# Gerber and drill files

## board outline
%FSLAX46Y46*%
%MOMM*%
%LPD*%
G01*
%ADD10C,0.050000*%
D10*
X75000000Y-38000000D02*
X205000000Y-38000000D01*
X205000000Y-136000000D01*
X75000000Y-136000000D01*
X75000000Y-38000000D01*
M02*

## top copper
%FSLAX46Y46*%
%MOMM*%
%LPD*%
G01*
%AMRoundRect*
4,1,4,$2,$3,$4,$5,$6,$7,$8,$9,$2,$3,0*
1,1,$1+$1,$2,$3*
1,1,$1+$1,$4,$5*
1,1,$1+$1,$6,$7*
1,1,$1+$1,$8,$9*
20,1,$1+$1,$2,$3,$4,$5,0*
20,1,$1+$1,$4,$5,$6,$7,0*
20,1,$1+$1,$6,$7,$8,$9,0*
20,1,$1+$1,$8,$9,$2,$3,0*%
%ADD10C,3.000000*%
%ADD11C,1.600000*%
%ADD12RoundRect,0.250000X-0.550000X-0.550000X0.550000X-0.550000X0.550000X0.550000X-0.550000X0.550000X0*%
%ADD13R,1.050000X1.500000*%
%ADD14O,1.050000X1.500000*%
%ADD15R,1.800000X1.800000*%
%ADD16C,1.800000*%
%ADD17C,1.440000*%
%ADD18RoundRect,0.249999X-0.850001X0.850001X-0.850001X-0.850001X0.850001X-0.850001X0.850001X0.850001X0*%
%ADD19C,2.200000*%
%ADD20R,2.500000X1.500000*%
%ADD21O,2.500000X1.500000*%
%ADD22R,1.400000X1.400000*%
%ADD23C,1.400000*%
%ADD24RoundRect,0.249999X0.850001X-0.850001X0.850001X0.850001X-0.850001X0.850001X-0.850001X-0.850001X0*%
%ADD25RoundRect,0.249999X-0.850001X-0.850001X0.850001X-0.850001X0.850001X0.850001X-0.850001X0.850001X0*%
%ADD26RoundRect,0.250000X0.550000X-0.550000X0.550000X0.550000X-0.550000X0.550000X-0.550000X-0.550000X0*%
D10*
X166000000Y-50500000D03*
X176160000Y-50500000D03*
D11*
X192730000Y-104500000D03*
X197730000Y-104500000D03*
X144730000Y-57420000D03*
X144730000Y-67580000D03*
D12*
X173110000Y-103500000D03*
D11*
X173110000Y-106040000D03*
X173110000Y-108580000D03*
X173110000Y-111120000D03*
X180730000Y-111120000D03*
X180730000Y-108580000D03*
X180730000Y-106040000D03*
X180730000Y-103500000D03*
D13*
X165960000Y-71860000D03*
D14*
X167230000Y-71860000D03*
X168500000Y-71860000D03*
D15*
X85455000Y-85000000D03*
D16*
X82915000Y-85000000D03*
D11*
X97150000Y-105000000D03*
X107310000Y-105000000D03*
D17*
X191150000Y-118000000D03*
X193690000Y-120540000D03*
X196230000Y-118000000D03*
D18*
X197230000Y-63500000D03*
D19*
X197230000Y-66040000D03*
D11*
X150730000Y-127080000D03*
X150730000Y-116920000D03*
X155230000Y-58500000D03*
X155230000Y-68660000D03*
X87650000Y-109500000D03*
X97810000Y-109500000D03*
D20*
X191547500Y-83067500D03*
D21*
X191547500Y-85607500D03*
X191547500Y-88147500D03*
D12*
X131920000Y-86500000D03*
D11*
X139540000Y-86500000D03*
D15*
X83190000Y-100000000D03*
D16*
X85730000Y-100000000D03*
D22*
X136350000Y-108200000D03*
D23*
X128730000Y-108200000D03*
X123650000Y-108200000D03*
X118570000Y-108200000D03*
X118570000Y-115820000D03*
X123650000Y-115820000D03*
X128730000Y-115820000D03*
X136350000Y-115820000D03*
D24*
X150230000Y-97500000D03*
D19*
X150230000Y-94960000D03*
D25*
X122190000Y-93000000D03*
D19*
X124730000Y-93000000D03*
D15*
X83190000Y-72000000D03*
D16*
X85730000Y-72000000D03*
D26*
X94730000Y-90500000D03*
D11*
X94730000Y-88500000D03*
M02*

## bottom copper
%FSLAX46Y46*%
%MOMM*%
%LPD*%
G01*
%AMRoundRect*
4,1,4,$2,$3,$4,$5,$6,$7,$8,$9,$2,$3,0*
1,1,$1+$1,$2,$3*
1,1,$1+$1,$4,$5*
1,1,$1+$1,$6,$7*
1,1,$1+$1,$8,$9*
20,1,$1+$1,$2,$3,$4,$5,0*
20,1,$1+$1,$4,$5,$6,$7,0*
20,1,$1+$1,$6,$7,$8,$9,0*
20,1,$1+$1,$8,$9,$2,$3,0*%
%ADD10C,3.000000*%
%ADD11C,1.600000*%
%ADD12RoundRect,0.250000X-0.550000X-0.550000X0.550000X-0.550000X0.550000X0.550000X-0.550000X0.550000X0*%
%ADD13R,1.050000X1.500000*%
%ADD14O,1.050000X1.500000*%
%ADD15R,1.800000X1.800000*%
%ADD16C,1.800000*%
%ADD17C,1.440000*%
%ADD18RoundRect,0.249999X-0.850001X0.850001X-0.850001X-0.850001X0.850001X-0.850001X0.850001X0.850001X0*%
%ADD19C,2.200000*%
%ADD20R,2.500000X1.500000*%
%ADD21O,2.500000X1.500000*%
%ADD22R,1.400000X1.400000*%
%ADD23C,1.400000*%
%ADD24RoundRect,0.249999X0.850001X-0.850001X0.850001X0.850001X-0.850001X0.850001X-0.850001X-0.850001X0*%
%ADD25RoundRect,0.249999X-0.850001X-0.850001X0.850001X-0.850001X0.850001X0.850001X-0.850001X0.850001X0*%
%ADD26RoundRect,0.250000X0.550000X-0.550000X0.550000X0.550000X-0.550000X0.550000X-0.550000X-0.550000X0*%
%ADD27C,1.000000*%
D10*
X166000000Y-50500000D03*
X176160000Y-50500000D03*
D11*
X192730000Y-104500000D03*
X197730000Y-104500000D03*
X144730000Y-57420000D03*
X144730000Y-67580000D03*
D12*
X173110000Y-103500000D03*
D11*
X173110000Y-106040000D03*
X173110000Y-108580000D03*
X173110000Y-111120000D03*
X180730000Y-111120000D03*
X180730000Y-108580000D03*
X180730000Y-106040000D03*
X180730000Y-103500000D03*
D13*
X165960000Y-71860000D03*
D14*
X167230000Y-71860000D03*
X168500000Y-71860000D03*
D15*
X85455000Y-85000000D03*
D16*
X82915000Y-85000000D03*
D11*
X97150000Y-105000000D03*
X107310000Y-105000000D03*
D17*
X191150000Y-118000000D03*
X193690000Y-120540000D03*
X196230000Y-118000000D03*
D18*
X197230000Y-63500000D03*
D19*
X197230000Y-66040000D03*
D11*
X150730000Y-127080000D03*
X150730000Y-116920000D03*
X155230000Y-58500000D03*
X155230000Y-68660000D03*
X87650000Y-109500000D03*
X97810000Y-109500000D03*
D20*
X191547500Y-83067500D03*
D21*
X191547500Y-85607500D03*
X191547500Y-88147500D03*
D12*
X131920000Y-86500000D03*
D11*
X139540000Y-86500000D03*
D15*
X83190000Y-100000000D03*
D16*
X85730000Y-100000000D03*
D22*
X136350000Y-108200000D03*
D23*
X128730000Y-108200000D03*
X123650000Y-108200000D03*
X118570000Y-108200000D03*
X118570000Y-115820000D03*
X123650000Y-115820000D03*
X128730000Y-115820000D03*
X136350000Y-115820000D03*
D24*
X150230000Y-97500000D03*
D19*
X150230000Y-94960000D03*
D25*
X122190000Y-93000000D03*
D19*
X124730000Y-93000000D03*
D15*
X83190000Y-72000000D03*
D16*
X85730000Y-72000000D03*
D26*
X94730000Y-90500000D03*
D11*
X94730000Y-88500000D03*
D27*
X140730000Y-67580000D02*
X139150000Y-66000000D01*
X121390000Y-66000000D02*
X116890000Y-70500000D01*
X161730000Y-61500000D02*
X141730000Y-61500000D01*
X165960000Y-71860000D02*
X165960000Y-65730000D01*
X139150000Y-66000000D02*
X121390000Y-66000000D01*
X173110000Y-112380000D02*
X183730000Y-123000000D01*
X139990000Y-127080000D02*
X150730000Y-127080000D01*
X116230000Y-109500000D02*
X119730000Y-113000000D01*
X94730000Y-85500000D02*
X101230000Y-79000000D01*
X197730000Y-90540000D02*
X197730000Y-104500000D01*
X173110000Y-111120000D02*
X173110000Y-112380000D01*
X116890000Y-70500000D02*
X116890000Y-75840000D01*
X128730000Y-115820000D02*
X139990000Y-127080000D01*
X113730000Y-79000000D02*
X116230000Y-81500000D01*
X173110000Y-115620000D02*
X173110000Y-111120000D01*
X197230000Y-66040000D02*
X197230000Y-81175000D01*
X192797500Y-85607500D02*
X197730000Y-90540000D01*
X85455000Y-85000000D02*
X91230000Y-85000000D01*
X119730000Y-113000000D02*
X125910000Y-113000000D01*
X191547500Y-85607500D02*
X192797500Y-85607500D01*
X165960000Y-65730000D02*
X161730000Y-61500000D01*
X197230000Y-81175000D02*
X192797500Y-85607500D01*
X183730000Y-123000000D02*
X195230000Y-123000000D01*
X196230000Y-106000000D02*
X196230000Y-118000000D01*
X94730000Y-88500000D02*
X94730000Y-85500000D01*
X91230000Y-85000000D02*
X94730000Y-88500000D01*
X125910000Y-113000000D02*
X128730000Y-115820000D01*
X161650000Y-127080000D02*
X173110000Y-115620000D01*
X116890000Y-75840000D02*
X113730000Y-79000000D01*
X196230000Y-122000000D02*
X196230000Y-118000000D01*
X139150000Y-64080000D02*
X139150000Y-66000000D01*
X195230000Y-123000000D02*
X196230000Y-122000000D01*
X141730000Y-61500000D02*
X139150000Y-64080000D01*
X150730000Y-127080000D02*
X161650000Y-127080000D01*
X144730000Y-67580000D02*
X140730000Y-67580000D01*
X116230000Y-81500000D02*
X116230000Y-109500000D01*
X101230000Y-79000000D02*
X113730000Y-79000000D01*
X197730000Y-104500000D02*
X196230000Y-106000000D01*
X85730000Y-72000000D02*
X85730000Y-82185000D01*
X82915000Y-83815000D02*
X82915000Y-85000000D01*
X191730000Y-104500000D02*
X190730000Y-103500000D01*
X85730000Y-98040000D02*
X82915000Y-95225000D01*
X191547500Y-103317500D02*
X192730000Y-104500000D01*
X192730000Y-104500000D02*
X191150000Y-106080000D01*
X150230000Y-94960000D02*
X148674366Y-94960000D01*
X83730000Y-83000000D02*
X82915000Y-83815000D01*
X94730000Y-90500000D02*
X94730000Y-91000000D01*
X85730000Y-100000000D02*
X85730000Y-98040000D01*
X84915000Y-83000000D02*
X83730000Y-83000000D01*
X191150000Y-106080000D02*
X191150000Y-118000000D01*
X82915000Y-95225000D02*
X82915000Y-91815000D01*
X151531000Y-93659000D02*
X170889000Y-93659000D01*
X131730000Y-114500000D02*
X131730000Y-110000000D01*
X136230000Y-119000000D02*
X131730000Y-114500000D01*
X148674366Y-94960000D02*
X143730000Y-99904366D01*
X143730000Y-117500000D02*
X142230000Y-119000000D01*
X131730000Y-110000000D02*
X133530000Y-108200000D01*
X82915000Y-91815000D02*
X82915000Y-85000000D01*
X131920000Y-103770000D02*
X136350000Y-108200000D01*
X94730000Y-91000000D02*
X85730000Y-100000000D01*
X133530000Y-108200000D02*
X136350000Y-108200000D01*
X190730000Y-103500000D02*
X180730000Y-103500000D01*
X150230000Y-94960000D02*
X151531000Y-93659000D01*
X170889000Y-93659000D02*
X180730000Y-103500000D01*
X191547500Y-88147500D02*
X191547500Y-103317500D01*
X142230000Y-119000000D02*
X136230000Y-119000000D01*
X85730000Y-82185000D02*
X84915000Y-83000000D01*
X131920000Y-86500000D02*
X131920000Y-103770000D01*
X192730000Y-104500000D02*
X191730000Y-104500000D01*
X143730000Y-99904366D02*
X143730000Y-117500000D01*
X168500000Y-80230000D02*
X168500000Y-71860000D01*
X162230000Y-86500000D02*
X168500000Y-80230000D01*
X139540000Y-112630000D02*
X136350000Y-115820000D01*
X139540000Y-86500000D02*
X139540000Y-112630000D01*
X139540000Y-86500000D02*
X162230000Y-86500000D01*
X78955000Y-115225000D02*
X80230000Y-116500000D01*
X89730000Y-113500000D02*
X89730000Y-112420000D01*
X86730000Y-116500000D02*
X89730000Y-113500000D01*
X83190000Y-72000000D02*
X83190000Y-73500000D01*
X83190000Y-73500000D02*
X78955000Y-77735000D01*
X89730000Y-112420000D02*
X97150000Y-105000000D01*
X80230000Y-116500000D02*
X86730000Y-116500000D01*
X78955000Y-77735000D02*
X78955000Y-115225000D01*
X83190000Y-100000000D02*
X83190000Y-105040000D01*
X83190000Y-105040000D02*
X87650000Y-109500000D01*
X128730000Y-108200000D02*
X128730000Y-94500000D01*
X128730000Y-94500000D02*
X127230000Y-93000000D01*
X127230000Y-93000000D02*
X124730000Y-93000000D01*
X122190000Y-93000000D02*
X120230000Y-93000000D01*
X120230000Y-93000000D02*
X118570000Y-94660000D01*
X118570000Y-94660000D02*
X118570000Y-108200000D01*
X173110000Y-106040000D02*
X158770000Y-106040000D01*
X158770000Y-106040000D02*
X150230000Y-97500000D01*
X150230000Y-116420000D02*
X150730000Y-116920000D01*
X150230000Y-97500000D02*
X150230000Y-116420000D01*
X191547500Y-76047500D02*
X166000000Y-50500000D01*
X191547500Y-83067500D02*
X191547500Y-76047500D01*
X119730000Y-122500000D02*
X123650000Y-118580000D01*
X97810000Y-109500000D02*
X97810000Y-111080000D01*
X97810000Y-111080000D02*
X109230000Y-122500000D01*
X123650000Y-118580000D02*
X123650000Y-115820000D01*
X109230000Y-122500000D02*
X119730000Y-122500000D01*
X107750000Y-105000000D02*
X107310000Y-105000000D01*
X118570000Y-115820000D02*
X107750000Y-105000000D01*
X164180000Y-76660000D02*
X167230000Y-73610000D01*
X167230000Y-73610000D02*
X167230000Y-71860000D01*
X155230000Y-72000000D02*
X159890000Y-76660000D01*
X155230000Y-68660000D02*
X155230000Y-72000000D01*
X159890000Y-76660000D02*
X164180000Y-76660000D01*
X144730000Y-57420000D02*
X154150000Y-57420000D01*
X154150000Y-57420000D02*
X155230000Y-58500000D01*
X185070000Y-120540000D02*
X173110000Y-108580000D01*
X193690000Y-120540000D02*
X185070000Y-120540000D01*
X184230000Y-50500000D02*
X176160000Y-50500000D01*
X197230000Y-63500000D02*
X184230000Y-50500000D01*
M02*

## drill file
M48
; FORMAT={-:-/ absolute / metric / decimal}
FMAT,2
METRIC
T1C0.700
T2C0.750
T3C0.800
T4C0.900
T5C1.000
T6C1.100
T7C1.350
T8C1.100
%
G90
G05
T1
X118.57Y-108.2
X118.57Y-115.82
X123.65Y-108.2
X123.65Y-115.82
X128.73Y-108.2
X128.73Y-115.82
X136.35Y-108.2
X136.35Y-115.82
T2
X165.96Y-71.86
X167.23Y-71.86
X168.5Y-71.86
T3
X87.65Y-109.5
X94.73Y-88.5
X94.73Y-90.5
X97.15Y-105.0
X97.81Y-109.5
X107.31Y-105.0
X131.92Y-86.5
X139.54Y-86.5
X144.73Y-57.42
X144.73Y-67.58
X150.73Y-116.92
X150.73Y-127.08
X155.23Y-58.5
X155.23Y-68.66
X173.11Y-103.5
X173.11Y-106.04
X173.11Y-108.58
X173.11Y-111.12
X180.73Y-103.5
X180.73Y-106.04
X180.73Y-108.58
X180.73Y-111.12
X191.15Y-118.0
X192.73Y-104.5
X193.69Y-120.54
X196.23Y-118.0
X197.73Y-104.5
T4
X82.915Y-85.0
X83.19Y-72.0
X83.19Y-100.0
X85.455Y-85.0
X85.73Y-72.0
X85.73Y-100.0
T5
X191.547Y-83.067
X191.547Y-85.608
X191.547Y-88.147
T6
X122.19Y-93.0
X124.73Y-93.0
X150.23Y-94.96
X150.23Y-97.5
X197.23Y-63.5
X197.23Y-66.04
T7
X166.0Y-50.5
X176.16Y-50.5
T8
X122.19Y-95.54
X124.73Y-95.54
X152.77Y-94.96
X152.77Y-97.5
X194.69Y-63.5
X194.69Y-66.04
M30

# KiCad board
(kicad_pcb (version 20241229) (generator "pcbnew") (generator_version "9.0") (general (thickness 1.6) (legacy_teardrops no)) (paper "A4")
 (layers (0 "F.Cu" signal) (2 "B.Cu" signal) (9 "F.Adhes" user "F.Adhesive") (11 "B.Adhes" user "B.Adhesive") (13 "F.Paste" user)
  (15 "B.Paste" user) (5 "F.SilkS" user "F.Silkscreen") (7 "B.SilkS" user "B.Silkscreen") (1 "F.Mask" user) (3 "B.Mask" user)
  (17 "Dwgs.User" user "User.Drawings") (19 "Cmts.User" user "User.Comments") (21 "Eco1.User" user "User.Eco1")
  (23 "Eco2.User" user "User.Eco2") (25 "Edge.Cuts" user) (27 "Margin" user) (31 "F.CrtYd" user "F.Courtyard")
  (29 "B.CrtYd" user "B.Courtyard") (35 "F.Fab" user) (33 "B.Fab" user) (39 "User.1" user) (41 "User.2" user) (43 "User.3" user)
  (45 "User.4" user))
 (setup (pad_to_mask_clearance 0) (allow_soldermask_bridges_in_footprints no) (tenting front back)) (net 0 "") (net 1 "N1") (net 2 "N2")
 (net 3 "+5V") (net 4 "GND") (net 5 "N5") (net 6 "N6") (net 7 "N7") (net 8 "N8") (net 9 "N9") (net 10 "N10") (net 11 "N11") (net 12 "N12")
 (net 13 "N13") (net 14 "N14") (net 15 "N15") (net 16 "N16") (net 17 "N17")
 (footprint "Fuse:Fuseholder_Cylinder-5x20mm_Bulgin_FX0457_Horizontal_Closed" (layer "F.Cu") (at 166 50.5)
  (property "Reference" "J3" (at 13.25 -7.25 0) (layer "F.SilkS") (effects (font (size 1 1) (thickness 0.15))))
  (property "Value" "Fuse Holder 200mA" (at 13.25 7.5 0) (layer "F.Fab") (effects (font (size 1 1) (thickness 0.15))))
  (pad "1" thru_hole circle (at 0 0) (size 3 3) (drill 1.35) (layers "*.Cu" "*.Mask") (remove_unused_layers no) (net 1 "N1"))
  (pad "2" thru_hole circle (at 10.16 0) (size 3 3) (drill 1.35) (layers "*.Cu" "*.Mask") (remove_unused_layers no) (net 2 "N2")))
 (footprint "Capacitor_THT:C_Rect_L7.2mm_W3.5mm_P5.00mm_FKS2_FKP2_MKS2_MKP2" (layer "F.Cu") (at 192.73 104.5)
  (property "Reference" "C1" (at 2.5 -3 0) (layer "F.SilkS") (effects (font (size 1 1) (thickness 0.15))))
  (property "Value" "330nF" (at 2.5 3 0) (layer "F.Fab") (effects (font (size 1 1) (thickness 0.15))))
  (pad "1" thru_hole circle (at 0 0) (size 1.6 1.6) (drill 0.8) (layers "*.Cu" "*.Mask") (remove_unused_layers no) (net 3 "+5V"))
  (pad "2" thru_hole circle (at 5 0) (size 1.6 1.6) (drill 0.8) (layers "*.Cu" "*.Mask") (remove_unused_layers no) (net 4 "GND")))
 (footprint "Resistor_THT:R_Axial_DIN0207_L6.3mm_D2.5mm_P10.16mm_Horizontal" (layer "F.Cu") (at 144.73 57.42 -90)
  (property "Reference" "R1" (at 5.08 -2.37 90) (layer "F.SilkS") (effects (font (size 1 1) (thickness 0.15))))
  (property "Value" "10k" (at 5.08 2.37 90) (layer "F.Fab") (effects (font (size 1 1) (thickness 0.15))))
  (pad "1" thru_hole circle (at 0 0 270) (size 1.6 1.6) (drill 0.8) (layers "*.Cu" "*.Mask") (remove_unused_layers no) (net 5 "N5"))
  (pad "2" thru_hole circle (at 10.16 0 270) (size 1.6 1.6) (drill 0.8) (layers "*.Cu" "*.Mask") (remove_unused_layers no) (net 4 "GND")))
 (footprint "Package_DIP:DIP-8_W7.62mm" (layer "F.Cu") (at 173.11 103.5)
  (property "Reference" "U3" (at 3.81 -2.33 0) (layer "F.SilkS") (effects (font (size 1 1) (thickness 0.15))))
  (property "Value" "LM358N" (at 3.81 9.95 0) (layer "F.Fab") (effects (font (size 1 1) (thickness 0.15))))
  (pad "1" thru_hole roundrect (at 0 0) (size 1.6 1.6) (drill 0.8) (layers "*.Cu" "*.Mask") (remove_unused_layers no)
   (roundrect_rratio 0.15625) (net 5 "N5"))
  (pad "2" thru_hole circle (at 0 2.54) (size 1.6 1.6) (drill 0.8) (layers "*.Cu" "*.Mask") (remove_unused_layers no) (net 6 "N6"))
  (pad "3" thru_hole circle (at 0 5.08) (size 1.6 1.6) (drill 0.8) (layers "*.Cu" "*.Mask") (remove_unused_layers no) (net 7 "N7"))
  (pad "4" thru_hole circle (at 0 7.62) (size 1.6 1.6) (drill 0.8) (layers "*.Cu" "*.Mask") (remove_unused_layers no) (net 4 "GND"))
  (pad "5" thru_hole circle (at 7.62 7.62) (size 1.6 1.6) (drill 0.8) (layers "*.Cu" "*.Mask") (remove_unused_layers no) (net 4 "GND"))
  (pad "6" thru_hole circle (at 7.62 5.08) (size 1.6 1.6) (drill 0.8) (layers "*.Cu" "*.Mask") (remove_unused_layers no) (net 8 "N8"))
  (pad "7" thru_hole circle (at 7.62 2.54) (size 1.6 1.6) (drill 0.8) (layers "*.Cu" "*.Mask") (remove_unused_layers no) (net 8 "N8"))
  (pad "8" thru_hole circle (at 7.62 0) (size 1.6 1.6) (drill 0.8) (layers "*.Cu" "*.Mask") (remove_unused_layers no) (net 3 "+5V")))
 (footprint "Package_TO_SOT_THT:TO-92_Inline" (layer "F.Cu") (at 165.96 71.86)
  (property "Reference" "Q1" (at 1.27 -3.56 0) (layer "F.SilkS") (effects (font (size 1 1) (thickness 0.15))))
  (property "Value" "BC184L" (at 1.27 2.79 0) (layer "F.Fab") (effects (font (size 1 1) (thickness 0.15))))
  (pad "1" thru_hole rect (at 0 0) (size 1.05 1.5) (drill 0.75) (layers "*.Cu" "*.Mask") (remove_unused_layers no) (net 4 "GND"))
  (pad "2" thru_hole oval (at 1.27 0) (size 1.05 1.5) (drill 0.75) (layers "*.Cu" "*.Mask") (remove_unused_layers no) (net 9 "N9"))
  (pad "3" thru_hole oval (at 2.54 0) (size 1.05 1.5) (drill 0.75) (layers "*.Cu" "*.Mask") (remove_unused_layers no) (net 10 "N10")))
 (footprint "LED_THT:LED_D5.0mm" (layer "F.Cu") (at 85.455 85 180)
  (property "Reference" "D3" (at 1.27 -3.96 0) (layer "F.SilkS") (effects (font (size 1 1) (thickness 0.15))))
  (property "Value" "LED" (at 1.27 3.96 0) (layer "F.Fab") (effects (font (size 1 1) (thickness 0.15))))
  (pad "1" thru_hole rect (at 0 0 180) (size 1.8 1.8) (drill 0.9) (layers "*.Cu" "*.Mask") (remove_unused_layers no) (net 4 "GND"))
  (pad "2" thru_hole circle (at 2.54 0 180) (size 1.8 1.8) (drill 0.9) (layers "*.Cu" "*.Mask") (remove_unused_layers no) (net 3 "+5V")))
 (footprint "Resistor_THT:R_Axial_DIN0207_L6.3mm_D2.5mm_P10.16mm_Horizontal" (layer "F.Cu") (at 97.15 105)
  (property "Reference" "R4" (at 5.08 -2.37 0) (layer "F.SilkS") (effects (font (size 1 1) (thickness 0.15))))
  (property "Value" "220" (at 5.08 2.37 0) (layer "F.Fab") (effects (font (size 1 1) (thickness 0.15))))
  (pad "1" thru_hole circle (at 0 0) (size 1.6 1.6) (drill 0.8) (layers "*.Cu" "*.Mask") (remove_unused_layers no) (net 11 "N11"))
  (pad "2" thru_hole circle (at 10.16 0) (size 1.6 1.6) (drill 0.8) (layers "*.Cu" "*.Mask") (remove_unused_layers no) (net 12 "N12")))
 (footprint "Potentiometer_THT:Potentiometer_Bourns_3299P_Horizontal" (layer "F.Cu") (at 191.15 118 90)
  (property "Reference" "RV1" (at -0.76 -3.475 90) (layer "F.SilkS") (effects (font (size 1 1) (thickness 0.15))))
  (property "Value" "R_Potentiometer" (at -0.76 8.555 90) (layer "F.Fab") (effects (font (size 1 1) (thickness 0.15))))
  (pad "1" thru_hole circle (at 0 0 90) (size 1.44 1.44) (drill 0.8) (layers "*.Cu" "*.Mask") (remove_unused_layers no) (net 3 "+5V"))
  (pad "2" thru_hole circle (at -2.54 2.54 90) (size 1.44 1.44) (drill 0.8) (layers "*.Cu" "*.Mask") (remove_unused_layers no) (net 7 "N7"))
  (pad "3" thru_hole circle (at 0 5.08 90) (size 1.44 1.44) (drill 0.8) (layers "*.Cu" "*.Mask") (remove_unused_layers no) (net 4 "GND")))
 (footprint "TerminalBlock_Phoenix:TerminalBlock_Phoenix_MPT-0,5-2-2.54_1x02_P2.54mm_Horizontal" (layer "F.Cu") (at 197.23 63.5 -90)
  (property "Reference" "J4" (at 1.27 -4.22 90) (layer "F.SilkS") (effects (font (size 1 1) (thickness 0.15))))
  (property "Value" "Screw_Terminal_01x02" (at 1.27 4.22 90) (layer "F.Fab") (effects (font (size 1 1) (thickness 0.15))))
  (pad "" np_thru_hole circle (at 0 2.54 270) (size 1.1 1.1) (drill 1.1) (layers "*.Cu" "*.Mask"))
  (pad "" np_thru_hole circle (at 2.54 2.54 270) (size 1.1 1.1) (drill 1.1) (layers "*.Cu" "*.Mask"))
  (pad "1" thru_hole roundrect (at 0 0 270) (size 2.2 2.2) (drill 1.1) (layers "*.Cu" "*.Mask") (remove_unused_layers no)
   (roundrect_rratio 0.113636) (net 2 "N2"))
  (pad "2" thru_hole circle (at 2.54 0 270) (size 2.2 2.2) (drill 1.1) (layers "*.Cu" "*.Mask") (remove_unused_layers no) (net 4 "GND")))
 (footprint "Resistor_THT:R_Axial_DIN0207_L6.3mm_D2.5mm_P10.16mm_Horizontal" (layer "F.Cu") (at 150.73 127.08 90)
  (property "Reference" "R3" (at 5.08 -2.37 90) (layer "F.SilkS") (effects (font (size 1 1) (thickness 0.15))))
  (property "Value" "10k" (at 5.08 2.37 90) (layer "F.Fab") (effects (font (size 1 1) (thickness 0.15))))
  (pad "1" thru_hole circle (at 0 0 90) (size 1.6 1.6) (drill 0.8) (layers "*.Cu" "*.Mask") (remove_unused_layers no) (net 4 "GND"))
  (pad "2" thru_hole circle (at 10.16 0 90) (size 1.6 1.6) (drill 0.8) (layers "*.Cu" "*.Mask") (remove_unused_layers no) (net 6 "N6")))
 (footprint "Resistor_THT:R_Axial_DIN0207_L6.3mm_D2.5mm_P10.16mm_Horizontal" (layer "F.Cu") (at 155.23 58.5 -90)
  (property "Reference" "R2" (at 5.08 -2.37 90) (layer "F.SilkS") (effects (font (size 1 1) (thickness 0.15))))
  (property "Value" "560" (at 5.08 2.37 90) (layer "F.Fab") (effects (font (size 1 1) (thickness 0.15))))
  (pad "1" thru_hole circle (at 0 0 270) (size 1.6 1.6) (drill 0.8) (layers "*.Cu" "*.Mask") (remove_unused_layers no) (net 5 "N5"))
  (pad "2" thru_hole circle (at 10.16 0 270) (size 1.6 1.6) (drill 0.8) (layers "*.Cu" "*.Mask") (remove_unused_layers no) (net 9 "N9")))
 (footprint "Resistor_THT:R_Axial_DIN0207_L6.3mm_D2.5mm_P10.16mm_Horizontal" (layer "F.Cu") (at 87.65 109.5)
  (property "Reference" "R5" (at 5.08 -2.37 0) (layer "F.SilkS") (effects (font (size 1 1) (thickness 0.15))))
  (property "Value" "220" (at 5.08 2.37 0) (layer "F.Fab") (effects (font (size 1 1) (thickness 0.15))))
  (pad "1" thru_hole circle (at 0 0) (size 1.6 1.6) (drill 0.8) (layers "*.Cu" "*.Mask") (remove_unused_layers no) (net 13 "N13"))
  (pad "2" thru_hole circle (at 10.16 0) (size 1.6 1.6) (drill 0.8) (layers "*.Cu" "*.Mask") (remove_unused_layers no) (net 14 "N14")))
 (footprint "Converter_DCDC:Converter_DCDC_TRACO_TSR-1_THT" (layer "F.Cu") (at 191.5475 83.0675 -90)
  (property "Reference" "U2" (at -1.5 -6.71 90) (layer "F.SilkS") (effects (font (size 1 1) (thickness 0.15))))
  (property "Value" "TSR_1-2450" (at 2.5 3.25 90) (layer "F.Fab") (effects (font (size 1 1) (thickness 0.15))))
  (pad "1" thru_hole rect (at 0 0 270) (size 1.5 2.5) (drill 1) (layers "*.Cu" "*.Mask") (remove_unused_layers no) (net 1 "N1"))
  (pad "2" thru_hole oval (at 2.54 0 270) (size 1.5 2.5) (drill 1) (layers "*.Cu" "*.Mask") (remove_unused_layers no) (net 4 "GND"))
  (pad "3" thru_hole oval (at 5.08 0 270) (size 1.5 2.5) (drill 1) (layers "*.Cu" "*.Mask") (remove_unused_layers no) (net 3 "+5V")))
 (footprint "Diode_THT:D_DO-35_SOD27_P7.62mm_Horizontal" (layer "F.Cu") (at 131.92 86.5)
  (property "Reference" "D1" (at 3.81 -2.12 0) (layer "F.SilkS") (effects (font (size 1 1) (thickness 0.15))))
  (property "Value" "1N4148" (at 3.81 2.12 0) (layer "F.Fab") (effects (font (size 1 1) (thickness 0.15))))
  (pad "1" thru_hole roundrect (at 0 0) (size 1.6 1.6) (drill 0.8) (layers "*.Cu" "*.Mask") (remove_unused_layers no)
   (roundrect_rratio 0.15625) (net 3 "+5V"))
  (pad "2" thru_hole circle (at 7.62 0) (size 1.6 1.6) (drill 0.8) (layers "*.Cu" "*.Mask") (remove_unused_layers no) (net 10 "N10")))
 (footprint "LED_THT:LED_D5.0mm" (layer "F.Cu") (at 83.19 100)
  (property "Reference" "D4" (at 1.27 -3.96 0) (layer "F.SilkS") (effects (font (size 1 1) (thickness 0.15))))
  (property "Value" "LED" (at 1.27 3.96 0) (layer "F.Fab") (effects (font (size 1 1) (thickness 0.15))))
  (pad "1" thru_hole rect (at 0 0) (size 1.8 1.8) (drill 0.9) (layers "*.Cu" "*.Mask") (remove_unused_layers no) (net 13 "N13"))
  (pad "2" thru_hole circle (at 2.54 0) (size 1.8 1.8) (drill 0.9) (layers "*.Cu" "*.Mask") (remove_unused_layers no) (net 3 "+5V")))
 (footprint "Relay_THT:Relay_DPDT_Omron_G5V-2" (layer "F.Cu") (at 136.35 108.2 -90)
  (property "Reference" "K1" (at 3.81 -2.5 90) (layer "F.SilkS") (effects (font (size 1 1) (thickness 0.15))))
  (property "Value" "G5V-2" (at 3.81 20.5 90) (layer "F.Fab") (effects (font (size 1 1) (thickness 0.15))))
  (pad "1" thru_hole rect (at 0 0 270) (size 1.4 1.4) (drill 0.7) (layers "*.Cu" "*.Mask") (remove_unused_layers no) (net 3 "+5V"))
  (pad "4" thru_hole circle (at 0 7.62 270) (size 1.4 1.4) (drill 0.7) (layers "*.Cu" "*.Mask") (remove_unused_layers no) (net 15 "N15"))
  (pad "6" thru_hole circle (at 0 12.7 270) (size 1.4 1.4) (drill 0.7) (layers "*.Cu" "*.Mask") (remove_unused_layers no) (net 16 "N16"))
  (pad "8" thru_hole circle (at 0 17.78 270) (size 1.4 1.4) (drill 0.7) (layers "*.Cu" "*.Mask") (remove_unused_layers no) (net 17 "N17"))
  (pad "9" thru_hole circle (at 7.62 17.78 270) (size 1.4 1.4) (drill 0.7) (layers "*.Cu" "*.Mask") (remove_unused_layers no) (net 12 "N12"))
  (pad "11" thru_hole circle (at 7.62 12.7 270) (size 1.4 1.4) (drill 0.7) (layers "*.Cu" "*.Mask") (remove_unused_layers no) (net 14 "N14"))
  (pad "13" thru_hole circle (at 7.62 7.62 270) (size 1.4 1.4) (drill 0.7) (layers "*.Cu" "*.Mask") (remove_unused_layers no) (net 4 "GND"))
  (pad "16" thru_hole circle (at 7.62 0 270) (size 1.4 1.4) (drill 0.7) (layers "*.Cu" "*.Mask") (remove_unused_layers no) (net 10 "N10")))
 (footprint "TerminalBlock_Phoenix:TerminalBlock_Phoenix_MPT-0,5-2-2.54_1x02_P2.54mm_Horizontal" (layer "F.Cu") (at 150.23 97.5 90)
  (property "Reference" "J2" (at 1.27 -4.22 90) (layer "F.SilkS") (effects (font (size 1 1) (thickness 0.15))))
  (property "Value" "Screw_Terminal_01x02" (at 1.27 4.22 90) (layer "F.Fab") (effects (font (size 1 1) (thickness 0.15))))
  (pad "" np_thru_hole circle (at 0 2.54 90) (size 1.1 1.1) (drill 1.1) (layers "*.Cu" "*.Mask"))
  (pad "" np_thru_hole circle (at 2.54 2.54 90) (size 1.1 1.1) (drill 1.1) (layers "*.Cu" "*.Mask"))
  (pad "1" thru_hole roundrect (at 0 0 90) (size 2.2 2.2) (drill 1.1) (layers "*.Cu" "*.Mask") (remove_unused_layers no)
   (roundrect_rratio 0.113636) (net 6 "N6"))
  (pad "2" thru_hole circle (at 2.54 0 90) (size 2.2 2.2) (drill 1.1) (layers "*.Cu" "*.Mask") (remove_unused_layers no) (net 3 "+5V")))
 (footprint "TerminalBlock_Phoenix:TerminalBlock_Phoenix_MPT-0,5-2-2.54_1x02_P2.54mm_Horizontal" (layer "F.Cu") (at 122.19 93)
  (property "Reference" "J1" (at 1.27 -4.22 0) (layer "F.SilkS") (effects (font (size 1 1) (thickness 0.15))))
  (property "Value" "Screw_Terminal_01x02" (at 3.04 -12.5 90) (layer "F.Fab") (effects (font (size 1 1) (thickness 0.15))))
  (pad "" np_thru_hole circle (at 0 2.54) (size 1.1 1.1) (drill 1.1) (layers "*.Cu" "*.Mask"))
  (pad "" np_thru_hole circle (at 2.54 2.54) (size 1.1 1.1) (drill 1.1) (layers "*.Cu" "*.Mask"))
  (pad "1" thru_hole roundrect (at 0 0) (size 2.2 2.2) (drill 1.1) (layers "*.Cu" "*.Mask") (remove_unused_layers no)
   (roundrect_rratio 0.113636) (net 17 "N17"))
  (pad "2" thru_hole circle (at 2.54 0) (size 2.2 2.2) (drill 1.1) (layers "*.Cu" "*.Mask") (remove_unused_layers no) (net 15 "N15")))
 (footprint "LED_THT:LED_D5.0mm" (layer "F.Cu") (at 83.19 72)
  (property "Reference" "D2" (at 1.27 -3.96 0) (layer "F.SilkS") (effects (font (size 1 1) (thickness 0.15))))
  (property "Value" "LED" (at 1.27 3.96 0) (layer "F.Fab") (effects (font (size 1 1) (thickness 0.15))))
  (pad "1" thru_hole rect (at 0 0) (size 1.8 1.8) (drill 0.9) (layers "*.Cu" "*.Mask") (remove_unused_layers no) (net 11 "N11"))
  (pad "2" thru_hole circle (at 2.54 0) (size 1.8 1.8) (drill 0.9) (layers "*.Cu" "*.Mask") (remove_unused_layers no) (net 3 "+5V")))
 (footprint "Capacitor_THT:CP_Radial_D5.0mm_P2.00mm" (layer "F.Cu") (at 94.73 90.5 90)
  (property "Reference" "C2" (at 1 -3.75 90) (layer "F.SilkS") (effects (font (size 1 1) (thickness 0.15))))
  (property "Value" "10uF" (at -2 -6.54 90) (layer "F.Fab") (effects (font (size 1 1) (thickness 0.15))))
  (pad "1" thru_hole roundrect (at 0 0 90) (size 1.6 1.6) (drill 0.8) (layers "*.Cu" "*.Mask") (remove_unused_layers no)
   (roundrect_rratio 0.15625) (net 3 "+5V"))
  (pad "2" thru_hole circle (at 2 0 90) (size 1.6 1.6) (drill 0.8) (layers "*.Cu" "*.Mask") (remove_unused_layers no) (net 4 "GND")))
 (gr_rect (start 75 38) (end 205 136) (stroke (width 0.05) (type solid)) (fill no) (layer "Edge.Cuts"))
 (segment (start 140.73 67.58) (end 139.15 66) (width 1) (layer "B.Cu") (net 4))
 (segment (start 121.39 66) (end 116.89 70.5) (width 1) (layer "B.Cu") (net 4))
 (segment (start 161.73 61.5) (end 141.73 61.5) (width 1) (layer "B.Cu") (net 4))
 (segment (start 165.96 71.86) (end 165.96 65.73) (width 1) (layer "B.Cu") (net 4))
 (segment (start 139.15 66) (end 121.39 66) (width 1) (layer "B.Cu") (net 4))
 (segment (start 173.11 112.38) (end 183.73 123) (width 1) (layer "B.Cu") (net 4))
 (segment (start 139.99 127.08) (end 150.73 127.08) (width 1) (layer "B.Cu") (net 4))
 (segment (start 116.23 109.5) (end 119.73 113) (width 1) (layer "B.Cu") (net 4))
 (segment (start 94.73 85.5) (end 101.23 79) (width 1) (layer "B.Cu") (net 4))
 (segment (start 197.73 90.54) (end 197.73 104.5) (width 1) (layer "B.Cu") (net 4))
 (segment (start 173.11 111.12) (end 173.11 112.38) (width 1) (layer "B.Cu") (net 4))
 (segment (start 116.89 70.5) (end 116.89 75.84) (width 1) (layer "B.Cu") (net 4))
 (segment (start 128.73 115.82) (end 139.99 127.08) (width 1) (layer "B.Cu") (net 4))
 (segment (start 113.73 79) (end 116.23 81.5) (width 1) (layer "B.Cu") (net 4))
 (segment (start 173.11 115.62) (end 173.11 111.12) (width 1) (layer "B.Cu") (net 4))
 (segment (start 197.23 66.04) (end 197.23 81.175) (width 1) (layer "B.Cu") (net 4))
 (segment (start 192.7975 85.6075) (end 197.73 90.54) (width 1) (layer "B.Cu") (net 4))
 (segment (start 85.455 85) (end 91.23 85) (width 1) (layer "B.Cu") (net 4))
 (segment (start 119.73 113) (end 125.91 113) (width 1) (layer "B.Cu") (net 4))
 (segment (start 191.5475 85.6075) (end 192.7975 85.6075) (width 1) (layer "B.Cu") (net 4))
 (segment (start 165.96 65.73) (end 161.73 61.5) (width 1) (layer "B.Cu") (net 4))
 (segment (start 197.23 81.175) (end 192.7975 85.6075) (width 1) (layer "B.Cu") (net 4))
 (segment (start 183.73 123) (end 195.23 123) (width 1) (layer "B.Cu") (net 4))
 (segment (start 196.23 106) (end 196.23 118) (width 1) (layer "B.Cu") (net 4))
 (segment (start 94.73 88.5) (end 94.73 85.5) (width 1) (layer "B.Cu") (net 4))
 (segment (start 91.23 85) (end 94.73 88.5) (width 1) (layer "B.Cu") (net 4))
 (segment (start 125.91 113) (end 128.73 115.82) (width 1) (layer "B.Cu") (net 4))
 (segment (start 161.65 127.08) (end 173.11 115.62) (width 1) (layer "B.Cu") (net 4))
 (segment (start 116.89 75.84) (end 113.73 79) (width 1) (layer "B.Cu") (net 4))
 (segment (start 196.23 122) (end 196.23 118) (width 1) (layer "B.Cu") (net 4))
 (segment (start 139.15 64.08) (end 139.15 66) (width 1) (layer "B.Cu") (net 4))
 (segment (start 195.23 123) (end 196.23 122) (width 1) (layer "B.Cu") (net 4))
 (segment (start 141.73 61.5) (end 139.15 64.08) (width 1) (layer "B.Cu") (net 4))
 (segment (start 150.73 127.08) (end 161.65 127.08) (width 1) (layer "B.Cu") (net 4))
 (segment (start 144.73 67.58) (end 140.73 67.58) (width 1) (layer "B.Cu") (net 4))
 (segment (start 116.23 81.5) (end 116.23 109.5) (width 1) (layer "B.Cu") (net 4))
 (segment (start 101.23 79) (end 113.73 79) (width 1) (layer "B.Cu") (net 4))
 (segment (start 197.73 104.5) (end 196.23 106) (width 1) (layer "B.Cu") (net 4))
 (segment (start 85.73 72) (end 85.73 82.185) (width 1) (layer "B.Cu") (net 3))
 (segment (start 82.915 83.815) (end 82.915 85) (width 1) (layer "B.Cu") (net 3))
 (segment (start 191.73 104.5) (end 190.73 103.5) (width 1) (layer "B.Cu") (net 3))
 (segment (start 85.73 98.04) (end 82.915 95.225) (width 1) (layer "B.Cu") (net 3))
 (segment (start 191.5475 103.3175) (end 192.73 104.5) (width 1) (layer "B.Cu") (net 3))
 (segment (start 192.73 104.5) (end 191.15 106.08) (width 1) (layer "B.Cu") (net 3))
 (segment (start 150.23 94.96) (end 148.674366 94.96) (width 1) (layer "B.Cu") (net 3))
 (segment (start 83.73 83) (end 82.915 83.815) (width 1) (layer "B.Cu") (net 3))
 (segment (start 94.73 90.5) (end 94.73 91) (width 1) (layer "B.Cu") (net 3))
 (segment (start 85.73 100) (end 85.73 98.04) (width 1) (layer "B.Cu") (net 3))
 (segment (start 84.915 83) (end 83.73 83) (width 1) (layer "B.Cu") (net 3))
 (segment (start 191.15 106.08) (end 191.15 118) (width 1) (layer "B.Cu") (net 3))
 (segment (start 82.915 95.225) (end 82.915 91.815) (width 1) (layer "B.Cu") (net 3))
 (segment (start 151.531 93.659) (end 170.889 93.659) (width 1) (layer "B.Cu") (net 3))
 (segment (start 131.73 114.5) (end 131.73 110) (width 1) (layer "B.Cu") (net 3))
 (segment (start 136.23 119) (end 131.73 114.5) (width 1) (layer "B.Cu") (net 3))
 (segment (start 148.674366 94.96) (end 143.73 99.904366) (width 1) (layer "B.Cu") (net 3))
 (segment (start 143.73 117.5) (end 142.23 119) (width 1) (layer "B.Cu") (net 3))
 (segment (start 131.73 110) (end 133.53 108.2) (width 1) (layer "B.Cu") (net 3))
 (segment (start 82.915 91.815) (end 82.915 85) (width 1) (layer "B.Cu") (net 3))
 (segment (start 131.92 103.77) (end 136.35 108.2) (width 1) (layer "B.Cu") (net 3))
 (segment (start 94.73 91) (end 85.73 100) (width 1) (layer "B.Cu") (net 3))
 (segment (start 133.53 108.2) (end 136.35 108.2) (width 1) (layer "B.Cu") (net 3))
 (segment (start 190.73 103.5) (end 180.73 103.5) (width 1) (layer "B.Cu") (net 3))
 (segment (start 150.23 94.96) (end 151.531 93.659) (width 1) (layer "B.Cu") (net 3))
 (segment (start 170.889 93.659) (end 180.73 103.5) (width 1) (layer "B.Cu") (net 3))
 (segment (start 191.5475 88.1475) (end 191.5475 103.3175) (width 1) (layer "B.Cu") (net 3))
 (segment (start 142.23 119) (end 136.23 119) (width 1) (layer "B.Cu") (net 3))
 (segment (start 85.73 82.185) (end 84.915 83) (width 1) (layer "B.Cu") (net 3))
 (segment (start 131.92 86.5) (end 131.92 103.77) (width 1) (layer "B.Cu") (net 3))
 (segment (start 192.73 104.5) (end 191.73 104.5) (width 1) (layer "B.Cu") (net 3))
 (segment (start 143.73 99.904366) (end 143.73 117.5) (width 1) (layer "B.Cu") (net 3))
 (segment (start 168.5 80.23) (end 168.5 71.86) (width 1) (layer "B.Cu") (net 10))
 (segment (start 162.23 86.5) (end 168.5 80.23) (width 1) (layer "B.Cu") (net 10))
 (segment (start 139.54 112.63) (end 136.35 115.82) (width 1) (layer "B.Cu") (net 10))
 (segment (start 139.54 86.5) (end 139.54 112.63) (width 1) (layer "B.Cu") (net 10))
 (segment (start 139.54 86.5) (end 162.23 86.5) (width 1) (layer "B.Cu") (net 10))
 (segment (start 78.955 115.225) (end 80.23 116.5) (width 1) (layer "B.Cu") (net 11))
 (segment (start 89.73 113.5) (end 89.73 112.42) (width 1) (layer "B.Cu") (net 11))
 (segment (start 86.73 116.5) (end 89.73 113.5) (width 1) (layer "B.Cu") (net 11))
 (segment (start 83.19 72) (end 83.19 73.5) (width 1) (layer "B.Cu") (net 11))
 (segment (start 83.19 73.5) (end 78.955 77.735) (width 1) (layer "B.Cu") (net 11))
 (segment (start 89.73 112.42) (end 97.15 105) (width 1) (layer "B.Cu") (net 11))
 (segment (start 80.23 116.5) (end 86.73 116.5) (width 1) (layer "B.Cu") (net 11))
 (segment (start 78.955 77.735) (end 78.955 115.225) (width 1) (layer "B.Cu") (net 11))
 (segment (start 83.19 100) (end 83.19 105.04) (width 1) (layer "B.Cu") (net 13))
 (segment (start 83.19 105.04) (end 87.65 109.5) (width 1) (layer "B.Cu") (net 13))
 (segment (start 128.73 108.2) (end 128.73 94.5) (width 1) (layer "B.Cu") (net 15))
 (segment (start 128.73 94.5) (end 127.23 93) (width 1) (layer "B.Cu") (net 15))
 (segment (start 127.23 93) (end 124.73 93) (width 1) (layer "B.Cu") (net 15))
 (segment (start 122.19 93) (end 120.23 93) (width 1) (layer "B.Cu") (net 17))
 (segment (start 120.23 93) (end 118.57 94.66) (width 1) (layer "B.Cu") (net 17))
 (segment (start 118.57 94.66) (end 118.57 108.2) (width 1) (layer "B.Cu") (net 17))
 (segment (start 173.11 106.04) (end 158.77 106.04) (width 1) (layer "B.Cu") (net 6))
 (segment (start 158.77 106.04) (end 150.23 97.5) (width 1) (layer "B.Cu") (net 6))
 (segment (start 150.23 116.42) (end 150.73 116.92) (width 1) (layer "B.Cu") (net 6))
 (segment (start 150.23 97.5) (end 150.23 116.42) (width 1) (layer "B.Cu") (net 6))
 (segment (start 191.5475 76.0475) (end 166 50.5) (width 1) (layer "B.Cu") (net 1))
 (segment (start 191.5475 83.0675) (end 191.5475 76.0475) (width 1) (layer "B.Cu") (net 1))
 (segment (start 119.73 122.5) (end 123.65 118.58) (width 1) (layer "B.Cu") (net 14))
 (segment (start 97.81 109.5) (end 97.81 111.08) (width 1) (layer "B.Cu") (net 14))
 (segment (start 97.81 111.08) (end 109.23 122.5) (width 1) (layer "B.Cu") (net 14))
 (segment (start 123.65 118.58) (end 123.65 115.82) (width 1) (layer "B.Cu") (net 14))
 (segment (start 109.23 122.5) (end 119.73 122.5) (width 1) (layer "B.Cu") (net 14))
 (segment (start 107.75 105) (end 107.31 105) (width 1) (layer "B.Cu") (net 12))
 (segment (start 118.57 115.82) (end 107.75 105) (width 1) (layer "B.Cu") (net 12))
 (segment (start 164.18 76.66) (end 167.23 73.61) (width 1) (layer "B.Cu") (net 9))
 (segment (start 167.23 73.61) (end 167.23 71.86) (width 1) (layer "B.Cu") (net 9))
 (segment (start 155.23 72) (end 159.89 76.66) (width 1) (layer "B.Cu") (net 9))
 (segment (start 155.23 68.66) (end 155.23 72) (width 1) (layer "B.Cu") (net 9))
 (segment (start 159.89 76.66) (end 164.18 76.66) (width 1) (layer "B.Cu") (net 9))
 (segment (start 144.73 57.42) (end 154.15 57.42) (width 1) (layer "B.Cu") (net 5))
 (segment (start 154.15 57.42) (end 155.23 58.5) (width 1) (layer "B.Cu") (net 5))
 (segment (start 185.07 120.54) (end 173.11 108.58) (width 1) (layer "B.Cu") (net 7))
 (segment (start 193.69 120.54) (end 185.07 120.54) (width 1) (layer "B.Cu") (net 7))
 (segment (start 184.23 50.5) (end 176.16 50.5) (width 1) (layer "B.Cu") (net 2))
 (segment (start 197.23 63.5) (end 184.23 50.5) (width 1) (layer "B.Cu") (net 2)))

